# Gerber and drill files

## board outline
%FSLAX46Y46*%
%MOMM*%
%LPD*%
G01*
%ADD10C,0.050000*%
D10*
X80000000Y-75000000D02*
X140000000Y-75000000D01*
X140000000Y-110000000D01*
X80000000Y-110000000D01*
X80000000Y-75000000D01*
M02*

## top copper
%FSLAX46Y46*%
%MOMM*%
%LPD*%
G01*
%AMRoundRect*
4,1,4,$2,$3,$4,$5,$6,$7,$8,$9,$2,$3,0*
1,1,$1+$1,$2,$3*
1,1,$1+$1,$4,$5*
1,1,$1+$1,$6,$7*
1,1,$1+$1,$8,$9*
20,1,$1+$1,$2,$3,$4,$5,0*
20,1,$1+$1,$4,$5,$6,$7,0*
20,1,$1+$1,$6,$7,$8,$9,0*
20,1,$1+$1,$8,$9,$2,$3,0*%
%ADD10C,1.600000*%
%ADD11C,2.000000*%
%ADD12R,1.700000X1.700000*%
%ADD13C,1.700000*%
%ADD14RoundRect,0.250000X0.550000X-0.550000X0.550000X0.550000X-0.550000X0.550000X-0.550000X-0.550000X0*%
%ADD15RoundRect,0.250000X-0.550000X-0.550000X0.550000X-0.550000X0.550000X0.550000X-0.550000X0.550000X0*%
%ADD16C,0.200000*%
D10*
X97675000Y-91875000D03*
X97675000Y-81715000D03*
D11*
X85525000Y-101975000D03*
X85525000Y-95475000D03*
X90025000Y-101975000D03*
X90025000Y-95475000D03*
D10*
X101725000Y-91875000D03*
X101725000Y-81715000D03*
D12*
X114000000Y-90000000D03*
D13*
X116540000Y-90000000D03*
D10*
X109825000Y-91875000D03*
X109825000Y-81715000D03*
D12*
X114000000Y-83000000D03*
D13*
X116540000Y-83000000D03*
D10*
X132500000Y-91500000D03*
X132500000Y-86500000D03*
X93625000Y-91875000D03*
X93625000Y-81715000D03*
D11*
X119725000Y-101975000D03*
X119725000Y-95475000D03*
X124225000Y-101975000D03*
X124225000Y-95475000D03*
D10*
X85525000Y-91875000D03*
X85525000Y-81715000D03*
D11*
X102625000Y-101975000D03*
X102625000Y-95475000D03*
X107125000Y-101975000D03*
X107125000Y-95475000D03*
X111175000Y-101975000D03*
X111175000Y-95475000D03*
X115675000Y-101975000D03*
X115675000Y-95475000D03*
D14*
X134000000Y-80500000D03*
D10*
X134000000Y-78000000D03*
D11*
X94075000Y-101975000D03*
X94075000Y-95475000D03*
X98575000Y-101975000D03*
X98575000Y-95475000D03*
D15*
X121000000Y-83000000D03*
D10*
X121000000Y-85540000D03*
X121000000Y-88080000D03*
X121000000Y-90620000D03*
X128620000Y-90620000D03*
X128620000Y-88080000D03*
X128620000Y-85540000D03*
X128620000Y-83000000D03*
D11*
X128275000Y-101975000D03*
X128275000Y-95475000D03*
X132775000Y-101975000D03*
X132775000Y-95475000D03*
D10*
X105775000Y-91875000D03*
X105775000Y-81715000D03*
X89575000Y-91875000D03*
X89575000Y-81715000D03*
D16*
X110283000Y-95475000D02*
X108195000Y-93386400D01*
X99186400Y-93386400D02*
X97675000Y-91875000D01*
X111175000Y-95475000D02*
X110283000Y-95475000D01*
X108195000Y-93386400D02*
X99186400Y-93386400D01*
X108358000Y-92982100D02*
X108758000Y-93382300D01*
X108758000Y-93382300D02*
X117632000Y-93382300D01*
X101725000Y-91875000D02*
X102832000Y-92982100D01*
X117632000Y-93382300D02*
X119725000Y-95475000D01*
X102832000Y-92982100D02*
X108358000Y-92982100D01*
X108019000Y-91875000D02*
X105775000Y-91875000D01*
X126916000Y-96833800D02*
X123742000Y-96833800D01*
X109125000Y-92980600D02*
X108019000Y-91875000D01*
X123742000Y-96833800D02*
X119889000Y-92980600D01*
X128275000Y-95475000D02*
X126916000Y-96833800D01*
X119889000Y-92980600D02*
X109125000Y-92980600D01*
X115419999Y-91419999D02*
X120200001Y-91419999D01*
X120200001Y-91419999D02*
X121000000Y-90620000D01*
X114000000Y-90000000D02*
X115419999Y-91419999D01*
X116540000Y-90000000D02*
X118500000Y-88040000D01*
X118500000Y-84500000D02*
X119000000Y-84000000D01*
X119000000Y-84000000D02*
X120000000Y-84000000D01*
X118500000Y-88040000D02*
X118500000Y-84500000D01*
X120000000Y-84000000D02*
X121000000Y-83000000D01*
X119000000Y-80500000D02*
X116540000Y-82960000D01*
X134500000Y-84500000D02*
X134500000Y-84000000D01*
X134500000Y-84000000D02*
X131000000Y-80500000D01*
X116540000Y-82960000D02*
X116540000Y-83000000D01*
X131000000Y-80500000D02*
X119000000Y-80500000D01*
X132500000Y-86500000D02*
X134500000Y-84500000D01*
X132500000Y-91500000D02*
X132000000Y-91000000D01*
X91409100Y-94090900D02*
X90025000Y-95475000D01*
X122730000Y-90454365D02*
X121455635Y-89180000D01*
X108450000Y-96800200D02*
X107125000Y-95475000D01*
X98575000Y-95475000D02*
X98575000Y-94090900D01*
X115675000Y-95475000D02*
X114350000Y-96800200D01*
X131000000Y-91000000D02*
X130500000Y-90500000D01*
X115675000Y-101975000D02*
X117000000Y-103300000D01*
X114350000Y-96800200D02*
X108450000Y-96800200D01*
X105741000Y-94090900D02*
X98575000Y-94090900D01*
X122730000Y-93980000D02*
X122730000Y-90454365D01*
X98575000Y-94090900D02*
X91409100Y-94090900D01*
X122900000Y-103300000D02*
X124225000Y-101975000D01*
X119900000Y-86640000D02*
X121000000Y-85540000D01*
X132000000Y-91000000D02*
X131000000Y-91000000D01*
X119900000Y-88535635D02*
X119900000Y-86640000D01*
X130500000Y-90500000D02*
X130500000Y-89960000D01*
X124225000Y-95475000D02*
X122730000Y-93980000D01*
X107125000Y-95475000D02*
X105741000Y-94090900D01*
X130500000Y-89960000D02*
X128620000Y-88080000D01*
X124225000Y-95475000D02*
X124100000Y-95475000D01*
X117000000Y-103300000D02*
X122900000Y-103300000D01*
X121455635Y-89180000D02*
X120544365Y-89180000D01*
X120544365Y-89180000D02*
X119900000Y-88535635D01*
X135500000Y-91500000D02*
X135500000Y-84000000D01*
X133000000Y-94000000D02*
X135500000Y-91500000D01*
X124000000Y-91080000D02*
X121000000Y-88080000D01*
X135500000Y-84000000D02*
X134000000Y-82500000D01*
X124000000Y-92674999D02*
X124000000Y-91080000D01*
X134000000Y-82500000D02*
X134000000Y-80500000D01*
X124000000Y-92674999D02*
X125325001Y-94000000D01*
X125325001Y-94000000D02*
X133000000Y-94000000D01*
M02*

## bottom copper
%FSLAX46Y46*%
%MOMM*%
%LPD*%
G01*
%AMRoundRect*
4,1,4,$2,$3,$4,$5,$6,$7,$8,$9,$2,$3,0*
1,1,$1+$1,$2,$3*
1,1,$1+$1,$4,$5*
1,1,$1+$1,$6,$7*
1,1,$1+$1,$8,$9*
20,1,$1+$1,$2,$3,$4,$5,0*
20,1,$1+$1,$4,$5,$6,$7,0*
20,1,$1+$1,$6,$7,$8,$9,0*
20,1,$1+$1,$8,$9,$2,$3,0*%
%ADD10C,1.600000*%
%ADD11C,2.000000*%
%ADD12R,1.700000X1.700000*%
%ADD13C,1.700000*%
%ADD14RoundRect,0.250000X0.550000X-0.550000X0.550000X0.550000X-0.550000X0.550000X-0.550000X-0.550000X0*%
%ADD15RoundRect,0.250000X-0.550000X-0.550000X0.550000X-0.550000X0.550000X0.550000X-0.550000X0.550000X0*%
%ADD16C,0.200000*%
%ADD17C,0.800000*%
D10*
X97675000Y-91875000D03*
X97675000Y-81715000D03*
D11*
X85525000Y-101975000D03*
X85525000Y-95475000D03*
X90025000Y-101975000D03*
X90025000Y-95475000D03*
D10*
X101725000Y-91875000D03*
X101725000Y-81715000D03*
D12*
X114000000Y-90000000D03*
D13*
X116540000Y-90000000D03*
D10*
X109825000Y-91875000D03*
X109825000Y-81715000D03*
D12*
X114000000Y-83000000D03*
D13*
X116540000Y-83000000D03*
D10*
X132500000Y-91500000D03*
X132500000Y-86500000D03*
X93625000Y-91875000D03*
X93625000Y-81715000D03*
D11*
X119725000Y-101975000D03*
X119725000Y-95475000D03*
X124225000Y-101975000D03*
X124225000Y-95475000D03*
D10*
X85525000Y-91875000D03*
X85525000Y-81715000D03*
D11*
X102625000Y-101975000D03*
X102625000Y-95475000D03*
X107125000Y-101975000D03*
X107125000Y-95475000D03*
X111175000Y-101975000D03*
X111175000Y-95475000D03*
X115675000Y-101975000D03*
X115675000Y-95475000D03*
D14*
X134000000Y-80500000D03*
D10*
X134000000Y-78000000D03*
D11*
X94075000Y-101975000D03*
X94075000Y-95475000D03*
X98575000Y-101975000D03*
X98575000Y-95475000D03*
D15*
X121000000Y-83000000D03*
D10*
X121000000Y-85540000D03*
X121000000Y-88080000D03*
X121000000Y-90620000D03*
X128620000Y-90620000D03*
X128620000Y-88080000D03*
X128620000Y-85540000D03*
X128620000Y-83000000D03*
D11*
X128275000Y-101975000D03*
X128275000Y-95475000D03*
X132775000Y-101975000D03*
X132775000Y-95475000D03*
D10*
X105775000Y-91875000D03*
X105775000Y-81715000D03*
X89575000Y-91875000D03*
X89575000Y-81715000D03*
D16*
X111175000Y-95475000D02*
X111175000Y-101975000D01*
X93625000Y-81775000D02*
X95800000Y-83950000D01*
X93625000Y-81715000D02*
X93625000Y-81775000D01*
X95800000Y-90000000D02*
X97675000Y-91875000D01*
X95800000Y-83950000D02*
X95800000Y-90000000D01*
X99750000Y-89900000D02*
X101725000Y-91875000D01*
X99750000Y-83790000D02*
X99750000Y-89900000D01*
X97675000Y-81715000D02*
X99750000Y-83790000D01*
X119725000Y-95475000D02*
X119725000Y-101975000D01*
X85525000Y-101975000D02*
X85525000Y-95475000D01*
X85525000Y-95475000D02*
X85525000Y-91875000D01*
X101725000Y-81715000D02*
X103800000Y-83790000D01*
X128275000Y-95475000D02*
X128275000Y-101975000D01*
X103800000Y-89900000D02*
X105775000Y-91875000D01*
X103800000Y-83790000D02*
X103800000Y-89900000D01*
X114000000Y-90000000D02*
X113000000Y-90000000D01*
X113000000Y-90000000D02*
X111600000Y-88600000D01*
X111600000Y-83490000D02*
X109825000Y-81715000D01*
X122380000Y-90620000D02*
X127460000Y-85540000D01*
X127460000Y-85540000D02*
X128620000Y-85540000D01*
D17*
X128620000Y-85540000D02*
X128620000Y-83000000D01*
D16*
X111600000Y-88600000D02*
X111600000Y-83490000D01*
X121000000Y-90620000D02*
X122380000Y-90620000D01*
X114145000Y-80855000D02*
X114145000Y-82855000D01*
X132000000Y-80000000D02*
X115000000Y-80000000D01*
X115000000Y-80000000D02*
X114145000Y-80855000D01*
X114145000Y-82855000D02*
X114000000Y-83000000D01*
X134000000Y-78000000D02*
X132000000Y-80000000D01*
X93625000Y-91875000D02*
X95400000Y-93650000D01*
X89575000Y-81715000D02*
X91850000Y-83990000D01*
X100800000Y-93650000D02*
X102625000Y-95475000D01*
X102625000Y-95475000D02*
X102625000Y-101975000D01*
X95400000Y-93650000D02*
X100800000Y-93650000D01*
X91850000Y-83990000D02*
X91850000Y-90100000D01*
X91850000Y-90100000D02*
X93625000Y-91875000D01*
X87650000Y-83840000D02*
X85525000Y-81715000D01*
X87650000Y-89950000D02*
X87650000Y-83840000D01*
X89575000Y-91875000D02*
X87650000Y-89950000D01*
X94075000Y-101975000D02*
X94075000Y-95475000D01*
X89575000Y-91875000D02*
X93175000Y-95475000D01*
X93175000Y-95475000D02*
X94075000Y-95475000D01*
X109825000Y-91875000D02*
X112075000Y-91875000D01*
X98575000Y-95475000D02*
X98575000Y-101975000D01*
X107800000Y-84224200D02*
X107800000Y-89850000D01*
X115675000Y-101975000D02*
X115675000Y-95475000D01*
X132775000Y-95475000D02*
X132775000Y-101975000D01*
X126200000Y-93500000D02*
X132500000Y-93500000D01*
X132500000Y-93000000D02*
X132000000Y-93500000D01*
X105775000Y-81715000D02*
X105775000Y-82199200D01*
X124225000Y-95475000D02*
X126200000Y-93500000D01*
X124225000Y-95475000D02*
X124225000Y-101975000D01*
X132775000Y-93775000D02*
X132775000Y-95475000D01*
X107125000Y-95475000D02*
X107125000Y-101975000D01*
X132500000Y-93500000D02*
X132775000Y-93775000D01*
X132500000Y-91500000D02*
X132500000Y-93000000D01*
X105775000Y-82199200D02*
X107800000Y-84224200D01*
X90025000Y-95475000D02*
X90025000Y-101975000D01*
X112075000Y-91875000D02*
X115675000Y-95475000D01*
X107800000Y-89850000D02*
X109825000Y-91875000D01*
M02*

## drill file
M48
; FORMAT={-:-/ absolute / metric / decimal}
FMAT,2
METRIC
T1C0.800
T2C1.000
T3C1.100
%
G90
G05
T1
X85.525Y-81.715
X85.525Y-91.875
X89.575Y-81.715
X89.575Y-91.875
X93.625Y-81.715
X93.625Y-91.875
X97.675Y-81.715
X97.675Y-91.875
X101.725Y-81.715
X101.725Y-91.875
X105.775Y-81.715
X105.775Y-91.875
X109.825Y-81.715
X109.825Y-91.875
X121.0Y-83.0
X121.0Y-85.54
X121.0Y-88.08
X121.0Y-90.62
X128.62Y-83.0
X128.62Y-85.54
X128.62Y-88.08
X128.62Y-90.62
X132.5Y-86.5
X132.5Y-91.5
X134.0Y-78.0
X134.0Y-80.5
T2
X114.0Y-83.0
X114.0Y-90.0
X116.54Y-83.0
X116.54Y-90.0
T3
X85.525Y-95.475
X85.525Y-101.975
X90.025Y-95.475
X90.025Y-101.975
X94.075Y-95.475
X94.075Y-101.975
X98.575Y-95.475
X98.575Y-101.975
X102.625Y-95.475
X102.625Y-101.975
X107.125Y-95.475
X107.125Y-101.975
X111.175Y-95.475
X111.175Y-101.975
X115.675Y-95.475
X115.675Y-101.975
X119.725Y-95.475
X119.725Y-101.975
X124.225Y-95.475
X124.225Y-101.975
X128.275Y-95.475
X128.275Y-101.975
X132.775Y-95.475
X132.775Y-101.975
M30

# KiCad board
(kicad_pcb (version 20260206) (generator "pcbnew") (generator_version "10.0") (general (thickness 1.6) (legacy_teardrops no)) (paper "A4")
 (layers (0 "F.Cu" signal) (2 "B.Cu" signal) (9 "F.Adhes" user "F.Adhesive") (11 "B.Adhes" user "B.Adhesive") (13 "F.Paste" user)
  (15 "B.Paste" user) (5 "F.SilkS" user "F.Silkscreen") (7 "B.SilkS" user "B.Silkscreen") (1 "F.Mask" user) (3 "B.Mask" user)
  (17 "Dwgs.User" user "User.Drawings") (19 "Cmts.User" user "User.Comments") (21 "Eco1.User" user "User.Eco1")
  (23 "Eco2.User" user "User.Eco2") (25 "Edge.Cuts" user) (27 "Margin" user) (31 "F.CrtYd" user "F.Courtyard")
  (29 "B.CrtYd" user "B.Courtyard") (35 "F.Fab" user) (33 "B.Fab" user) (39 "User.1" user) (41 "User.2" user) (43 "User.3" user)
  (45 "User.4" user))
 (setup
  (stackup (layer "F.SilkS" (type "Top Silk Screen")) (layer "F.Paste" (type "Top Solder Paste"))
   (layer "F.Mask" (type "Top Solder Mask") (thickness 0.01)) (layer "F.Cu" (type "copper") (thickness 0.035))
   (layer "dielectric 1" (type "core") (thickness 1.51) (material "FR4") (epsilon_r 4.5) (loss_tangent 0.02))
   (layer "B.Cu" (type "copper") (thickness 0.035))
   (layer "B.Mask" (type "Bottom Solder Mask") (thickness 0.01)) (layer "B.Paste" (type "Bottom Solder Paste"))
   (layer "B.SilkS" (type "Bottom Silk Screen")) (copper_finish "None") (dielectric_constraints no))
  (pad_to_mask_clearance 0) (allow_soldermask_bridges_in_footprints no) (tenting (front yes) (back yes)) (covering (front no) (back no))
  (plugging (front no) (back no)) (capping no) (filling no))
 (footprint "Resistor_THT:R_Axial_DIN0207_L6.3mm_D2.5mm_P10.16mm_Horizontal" (layer "F.Cu") (at 97.675 91.875 90)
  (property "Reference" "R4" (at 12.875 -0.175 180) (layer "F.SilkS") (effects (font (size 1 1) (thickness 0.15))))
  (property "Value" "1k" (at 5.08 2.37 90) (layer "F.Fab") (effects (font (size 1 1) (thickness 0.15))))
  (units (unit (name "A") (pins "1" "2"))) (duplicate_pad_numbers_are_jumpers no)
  (pad "1" thru_hole circle (at 0 0 90) (size 1.6 1.6) (drill 0.8) (layers "*.Cu" "*.Mask") (remove_unused_layers no) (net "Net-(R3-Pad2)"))
  (pad "2" thru_hole circle (at 10.16 0 90) (size 1.6 1.6) (drill 0.8) (layers "*.Cu" "*.Mask") (remove_unused_layers no)
   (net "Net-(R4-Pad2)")))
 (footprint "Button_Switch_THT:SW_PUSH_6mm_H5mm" (layer "F.Cu") (at 85.525 101.975 90)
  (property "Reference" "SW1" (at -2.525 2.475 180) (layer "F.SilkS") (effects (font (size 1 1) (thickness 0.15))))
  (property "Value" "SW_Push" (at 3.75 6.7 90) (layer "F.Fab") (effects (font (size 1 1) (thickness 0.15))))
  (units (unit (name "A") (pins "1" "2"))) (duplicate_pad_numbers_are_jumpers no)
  (pad "1" thru_hole circle (at 0 0 180) (size 2 2) (drill 1.1) (layers "*.Cu" "*.Mask") (remove_unused_layers no) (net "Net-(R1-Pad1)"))
  (pad "1" thru_hole circle (at 6.5 0 180) (size 2 2) (drill 1.1) (layers "*.Cu" "*.Mask") (remove_unused_layers no) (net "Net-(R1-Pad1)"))
  (pad "2" thru_hole circle (at 0 4.5 180) (size 2 2) (drill 1.1) (layers "*.Cu" "*.Mask") (remove_unused_layers no) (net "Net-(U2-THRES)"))
  (pad "2" thru_hole circle (at 6.5 4.5 180) (size 2 2) (drill 1.1) (layers "*.Cu" "*.Mask") (remove_unused_layers no)
   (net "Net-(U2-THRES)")))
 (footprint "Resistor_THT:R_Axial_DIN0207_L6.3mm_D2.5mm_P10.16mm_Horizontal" (layer "F.Cu") (at 101.725 91.875 90)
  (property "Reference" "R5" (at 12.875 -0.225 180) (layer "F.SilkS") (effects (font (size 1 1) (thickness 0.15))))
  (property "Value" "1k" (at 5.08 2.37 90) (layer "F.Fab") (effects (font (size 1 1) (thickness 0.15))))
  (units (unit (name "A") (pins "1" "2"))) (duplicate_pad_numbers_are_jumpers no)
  (pad "1" thru_hole circle (at 0 0 90) (size 1.6 1.6) (drill 0.8) (layers "*.Cu" "*.Mask") (remove_unused_layers no) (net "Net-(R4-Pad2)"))
  (pad "2" thru_hole circle (at 10.16 0 90) (size 1.6 1.6) (drill 0.8) (layers "*.Cu" "*.Mask") (remove_unused_layers no)
   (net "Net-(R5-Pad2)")))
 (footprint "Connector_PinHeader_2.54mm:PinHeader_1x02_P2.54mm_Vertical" (layer "F.Cu") (at 114 90 90)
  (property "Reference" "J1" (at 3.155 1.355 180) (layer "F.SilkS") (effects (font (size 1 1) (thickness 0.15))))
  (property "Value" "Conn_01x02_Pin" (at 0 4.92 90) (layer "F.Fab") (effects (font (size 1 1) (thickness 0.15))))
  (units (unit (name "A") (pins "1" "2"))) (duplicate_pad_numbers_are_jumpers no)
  (pad "1" thru_hole rect (at 0 0 90) (size 1.7 1.7) (drill 1) (layers "*.Cu" "*.Mask") (remove_unused_layers no) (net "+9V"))
  (pad "2" thru_hole circle (at 0 2.54 90) (size 1.7 1.7) (drill 1) (layers "*.Cu" "*.Mask") (remove_unused_layers no) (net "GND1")))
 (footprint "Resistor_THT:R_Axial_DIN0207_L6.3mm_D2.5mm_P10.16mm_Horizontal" (layer "F.Cu") (at 109.825 91.875 90)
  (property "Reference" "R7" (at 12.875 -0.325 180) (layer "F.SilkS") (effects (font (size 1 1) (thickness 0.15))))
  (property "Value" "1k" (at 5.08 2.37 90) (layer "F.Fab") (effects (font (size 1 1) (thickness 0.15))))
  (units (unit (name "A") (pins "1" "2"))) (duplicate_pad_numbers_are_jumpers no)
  (pad "1" thru_hole circle (at 0 0 90) (size 1.6 1.6) (drill 0.8) (layers "*.Cu" "*.Mask") (remove_unused_layers no) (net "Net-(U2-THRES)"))
  (pad "2" thru_hole circle (at 10.16 0 90) (size 1.6 1.6) (drill 0.8) (layers "*.Cu" "*.Mask") (remove_unused_layers no) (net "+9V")))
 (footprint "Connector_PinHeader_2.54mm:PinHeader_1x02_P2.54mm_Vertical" (layer "F.Cu") (at 114 83 90)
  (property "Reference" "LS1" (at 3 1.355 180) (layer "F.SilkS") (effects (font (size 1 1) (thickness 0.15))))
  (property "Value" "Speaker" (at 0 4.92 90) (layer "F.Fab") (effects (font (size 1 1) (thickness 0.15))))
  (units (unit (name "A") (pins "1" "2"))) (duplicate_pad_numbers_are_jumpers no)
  (pad "1" thru_hole rect (at 0 0 90) (size 1.7 1.7) (drill 1) (layers "*.Cu" "*.Mask") (remove_unused_layers no) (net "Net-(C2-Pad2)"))
  (pad "2" thru_hole circle (at 0 2.54 90) (size 1.7 1.7) (drill 1) (layers "*.Cu" "*.Mask") (remove_unused_layers no) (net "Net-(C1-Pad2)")))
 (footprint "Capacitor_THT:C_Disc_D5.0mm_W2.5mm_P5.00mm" (layer "F.Cu") (at 132.5 91.5 90)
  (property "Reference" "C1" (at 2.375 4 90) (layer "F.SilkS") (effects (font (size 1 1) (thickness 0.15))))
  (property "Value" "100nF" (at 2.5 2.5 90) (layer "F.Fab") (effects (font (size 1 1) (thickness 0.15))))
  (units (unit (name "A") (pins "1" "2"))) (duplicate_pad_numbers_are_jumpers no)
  (pad "1" thru_hole circle (at 0 0 90) (size 1.6 1.6) (drill 0.8) (layers "*.Cu" "*.Mask") (remove_unused_layers no) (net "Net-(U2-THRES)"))
  (pad "2" thru_hole circle (at 5 0 90) (size 1.6 1.6) (drill 0.8) (layers "*.Cu" "*.Mask") (remove_unused_layers no) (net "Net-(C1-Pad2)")))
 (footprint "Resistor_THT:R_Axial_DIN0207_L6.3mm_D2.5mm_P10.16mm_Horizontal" (layer "F.Cu") (at 93.625 91.875 90)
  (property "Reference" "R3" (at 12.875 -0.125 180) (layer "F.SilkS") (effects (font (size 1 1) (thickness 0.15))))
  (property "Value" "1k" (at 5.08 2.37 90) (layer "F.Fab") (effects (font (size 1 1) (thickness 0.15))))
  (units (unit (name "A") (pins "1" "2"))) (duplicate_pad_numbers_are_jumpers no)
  (pad "1" thru_hole circle (at 0 0 90) (size 1.6 1.6) (drill 0.8) (layers "*.Cu" "*.Mask") (remove_unused_layers no) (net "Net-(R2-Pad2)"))
  (pad "2" thru_hole circle (at 10.16 0 90) (size 1.6 1.6) (drill 0.8) (layers "*.Cu" "*.Mask") (remove_unused_layers no)
   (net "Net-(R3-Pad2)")))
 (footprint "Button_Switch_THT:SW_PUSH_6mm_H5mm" (layer "F.Cu") (at 119.725 101.975 90)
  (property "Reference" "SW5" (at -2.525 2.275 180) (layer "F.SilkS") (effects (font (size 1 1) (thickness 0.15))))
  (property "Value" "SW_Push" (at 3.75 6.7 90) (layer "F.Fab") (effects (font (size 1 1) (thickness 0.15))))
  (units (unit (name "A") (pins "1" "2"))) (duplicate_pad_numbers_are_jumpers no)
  (pad "1" thru_hole circle (at 0 0 180) (size 2 2) (drill 1.1) (layers "*.Cu" "*.Mask") (remove_unused_layers no) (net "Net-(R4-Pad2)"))
  (pad "1" thru_hole circle (at 6.5 0 180) (size 2 2) (drill 1.1) (layers "*.Cu" "*.Mask") (remove_unused_layers no) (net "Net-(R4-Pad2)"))
  (pad "2" thru_hole circle (at 0 4.5 180) (size 2 2) (drill 1.1) (layers "*.Cu" "*.Mask") (remove_unused_layers no) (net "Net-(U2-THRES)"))
  (pad "2" thru_hole circle (at 6.5 4.5 180) (size 2 2) (drill 1.1) (layers "*.Cu" "*.Mask") (remove_unused_layers no)
   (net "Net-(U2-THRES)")))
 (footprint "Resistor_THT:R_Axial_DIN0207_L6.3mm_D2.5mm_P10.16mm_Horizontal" (layer "F.Cu") (at 85.525 91.875 90)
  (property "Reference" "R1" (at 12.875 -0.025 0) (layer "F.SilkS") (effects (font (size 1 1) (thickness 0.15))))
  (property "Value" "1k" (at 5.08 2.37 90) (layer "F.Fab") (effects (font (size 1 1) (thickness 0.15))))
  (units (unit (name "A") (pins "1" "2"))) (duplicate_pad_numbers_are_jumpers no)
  (pad "1" thru_hole circle (at 0 0 90) (size 1.6 1.6) (drill 0.8) (layers "*.Cu" "*.Mask") (remove_unused_layers no) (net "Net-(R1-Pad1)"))
  (pad "2" thru_hole circle (at 10.16 0 90) (size 1.6 1.6) (drill 0.8) (layers "*.Cu" "*.Mask") (remove_unused_layers no)
   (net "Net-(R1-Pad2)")))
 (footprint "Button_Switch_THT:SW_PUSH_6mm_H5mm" (layer "F.Cu") (at 102.625 101.975 90)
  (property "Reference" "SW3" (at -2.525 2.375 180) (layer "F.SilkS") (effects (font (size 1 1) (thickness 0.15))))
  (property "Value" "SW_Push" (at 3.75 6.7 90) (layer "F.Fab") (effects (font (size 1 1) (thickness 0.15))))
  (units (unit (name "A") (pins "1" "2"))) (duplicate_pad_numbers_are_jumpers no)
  (pad "1" thru_hole circle (at 0 0 180) (size 2 2) (drill 1.1) (layers "*.Cu" "*.Mask") (remove_unused_layers no) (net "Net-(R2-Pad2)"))
  (pad "1" thru_hole circle (at 6.5 0 180) (size 2 2) (drill 1.1) (layers "*.Cu" "*.Mask") (remove_unused_layers no) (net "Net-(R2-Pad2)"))
  (pad "2" thru_hole circle (at 0 4.5 180) (size 2 2) (drill 1.1) (layers "*.Cu" "*.Mask") (remove_unused_layers no) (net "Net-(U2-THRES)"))
  (pad "2" thru_hole circle (at 6.5 4.5 180) (size 2 2) (drill 1.1) (layers "*.Cu" "*.Mask") (remove_unused_layers no)
   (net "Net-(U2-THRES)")))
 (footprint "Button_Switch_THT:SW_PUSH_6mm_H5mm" (layer "F.Cu") (at 111.175 101.975 90)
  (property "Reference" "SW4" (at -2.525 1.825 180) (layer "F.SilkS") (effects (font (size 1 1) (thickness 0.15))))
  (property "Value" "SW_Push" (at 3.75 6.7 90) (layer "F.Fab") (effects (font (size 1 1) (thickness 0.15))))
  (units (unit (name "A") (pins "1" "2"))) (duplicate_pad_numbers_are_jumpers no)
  (pad "1" thru_hole circle (at 0 0 180) (size 2 2) (drill 1.1) (layers "*.Cu" "*.Mask") (remove_unused_layers no) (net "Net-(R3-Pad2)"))
  (pad "1" thru_hole circle (at 6.5 0 180) (size 2 2) (drill 1.1) (layers "*.Cu" "*.Mask") (remove_unused_layers no) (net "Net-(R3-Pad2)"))
  (pad "2" thru_hole circle (at 0 4.5 180) (size 2 2) (drill 1.1) (layers "*.Cu" "*.Mask") (remove_unused_layers no) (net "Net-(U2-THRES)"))
  (pad "2" thru_hole circle (at 6.5 4.5 180) (size 2 2) (drill 1.1) (layers "*.Cu" "*.Mask") (remove_unused_layers no)
   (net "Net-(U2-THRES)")))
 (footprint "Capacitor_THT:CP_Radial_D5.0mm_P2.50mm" (layer "F.Cu") (at 134 80.5 90)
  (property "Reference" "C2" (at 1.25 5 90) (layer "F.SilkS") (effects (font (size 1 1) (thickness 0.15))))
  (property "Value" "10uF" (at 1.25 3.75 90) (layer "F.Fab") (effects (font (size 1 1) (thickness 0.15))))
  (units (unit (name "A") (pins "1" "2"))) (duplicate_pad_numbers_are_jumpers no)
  (pad "1" thru_hole roundrect (at 0 0 90) (size 1.6 1.6) (drill 0.8) (layers "*.Cu" "*.Mask") (remove_unused_layers no)
   (roundrect_rratio 0.15625) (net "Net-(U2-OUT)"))
  (pad "2" thru_hole circle (at 2.5 0 90) (size 1.6 1.6) (drill 0.8) (layers "*.Cu" "*.Mask") (remove_unused_layers no)
   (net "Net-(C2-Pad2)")))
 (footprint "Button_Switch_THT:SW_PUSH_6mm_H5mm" (layer "F.Cu") (at 94.075 101.975 90)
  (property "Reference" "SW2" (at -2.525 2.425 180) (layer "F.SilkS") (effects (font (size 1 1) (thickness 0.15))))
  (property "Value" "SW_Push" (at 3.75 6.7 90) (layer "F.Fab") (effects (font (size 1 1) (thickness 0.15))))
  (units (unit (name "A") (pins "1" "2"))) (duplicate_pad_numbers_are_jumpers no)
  (pad "1" thru_hole circle (at 0 0 180) (size 2 2) (drill 1.1) (layers "*.Cu" "*.Mask") (remove_unused_layers no) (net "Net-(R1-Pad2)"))
  (pad "1" thru_hole circle (at 6.5 0 180) (size 2 2) (drill 1.1) (layers "*.Cu" "*.Mask") (remove_unused_layers no) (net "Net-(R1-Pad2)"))
  (pad "2" thru_hole circle (at 0 4.5 180) (size 2 2) (drill 1.1) (layers "*.Cu" "*.Mask") (remove_unused_layers no) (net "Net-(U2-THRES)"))
  (pad "2" thru_hole circle (at 6.5 4.5 180) (size 2 2) (drill 1.1) (layers "*.Cu" "*.Mask") (remove_unused_layers no)
   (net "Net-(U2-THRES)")))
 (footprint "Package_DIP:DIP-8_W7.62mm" (layer "F.Cu") (at 121 83)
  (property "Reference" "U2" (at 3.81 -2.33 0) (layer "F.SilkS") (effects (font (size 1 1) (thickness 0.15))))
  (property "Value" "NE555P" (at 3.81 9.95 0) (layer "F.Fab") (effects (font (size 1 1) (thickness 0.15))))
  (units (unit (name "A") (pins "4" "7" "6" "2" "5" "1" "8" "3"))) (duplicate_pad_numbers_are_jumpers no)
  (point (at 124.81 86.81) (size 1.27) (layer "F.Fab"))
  (pad "1" thru_hole roundrect (at 0 0) (size 1.6 1.6) (drill 0.8) (layers "*.Cu" "*.Mask") (remove_unused_layers no)
   (roundrect_rratio 0.15625) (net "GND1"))
  (pad "2" thru_hole circle (at 0 2.54) (size 1.6 1.6) (drill 0.8) (layers "*.Cu" "*.Mask") (remove_unused_layers no) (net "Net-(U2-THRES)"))
  (pad "3" thru_hole circle (at 0 5.08) (size 1.6 1.6) (drill 0.8) (layers "*.Cu" "*.Mask") (remove_unused_layers no) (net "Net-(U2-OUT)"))
  (pad "4" thru_hole circle (at 0 7.62) (size 1.6 1.6) (drill 0.8) (layers "*.Cu" "*.Mask") (remove_unused_layers no) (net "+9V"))
  (pad "5" thru_hole circle (at 7.62 7.62) (size 1.6 1.6) (drill 0.8) (layers "*.Cu" "*.Mask") (remove_unused_layers no)
   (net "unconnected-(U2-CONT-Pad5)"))
  (pad "6" thru_hole circle (at 7.62 5.08) (size 1.6 1.6) (drill 0.8) (layers "*.Cu" "*.Mask") (remove_unused_layers no)
   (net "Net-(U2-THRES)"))
  (pad "7" thru_hole circle (at 7.62 2.54) (size 1.6 1.6) (drill 0.8) (layers "*.Cu" "*.Mask") (remove_unused_layers no) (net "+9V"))
  (pad "8" thru_hole circle (at 7.62 0) (size 1.6 1.6) (drill 0.8) (layers "*.Cu" "*.Mask") (remove_unused_layers no) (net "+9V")))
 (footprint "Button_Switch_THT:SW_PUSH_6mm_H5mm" (layer "F.Cu") (at 128.275 101.975 90)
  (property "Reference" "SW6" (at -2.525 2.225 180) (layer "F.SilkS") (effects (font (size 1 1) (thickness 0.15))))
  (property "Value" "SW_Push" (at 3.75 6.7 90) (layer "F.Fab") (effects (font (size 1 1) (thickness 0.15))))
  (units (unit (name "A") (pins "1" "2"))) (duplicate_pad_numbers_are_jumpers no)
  (pad "1" thru_hole circle (at 0 0 180) (size 2 2) (drill 1.1) (layers "*.Cu" "*.Mask") (remove_unused_layers no) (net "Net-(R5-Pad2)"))
  (pad "1" thru_hole circle (at 6.5 0 180) (size 2 2) (drill 1.1) (layers "*.Cu" "*.Mask") (remove_unused_layers no) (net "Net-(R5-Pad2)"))
  (pad "2" thru_hole circle (at 0 4.5 180) (size 2 2) (drill 1.1) (layers "*.Cu" "*.Mask") (remove_unused_layers no) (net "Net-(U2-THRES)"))
  (pad "2" thru_hole circle (at 6.5 4.5 180) (size 2 2) (drill 1.1) (layers "*.Cu" "*.Mask") (remove_unused_layers no)
   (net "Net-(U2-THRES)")))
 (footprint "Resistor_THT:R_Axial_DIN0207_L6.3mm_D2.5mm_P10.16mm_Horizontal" (layer "F.Cu") (at 105.775 91.875 90)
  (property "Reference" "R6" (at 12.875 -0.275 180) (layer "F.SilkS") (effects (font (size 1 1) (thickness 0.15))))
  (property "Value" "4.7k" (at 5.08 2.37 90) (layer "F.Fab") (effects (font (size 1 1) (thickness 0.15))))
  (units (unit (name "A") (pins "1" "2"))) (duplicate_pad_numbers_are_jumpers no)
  (pad "1" thru_hole circle (at 0 0 90) (size 1.6 1.6) (drill 0.8) (layers "*.Cu" "*.Mask") (remove_unused_layers no) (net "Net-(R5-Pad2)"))
  (pad "2" thru_hole circle (at 10.16 0 90) (size 1.6 1.6) (drill 0.8) (layers "*.Cu" "*.Mask") (remove_unused_layers no)
   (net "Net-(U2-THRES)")))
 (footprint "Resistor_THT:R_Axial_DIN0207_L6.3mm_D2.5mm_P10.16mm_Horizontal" (layer "F.Cu") (at 89.575 91.875 90)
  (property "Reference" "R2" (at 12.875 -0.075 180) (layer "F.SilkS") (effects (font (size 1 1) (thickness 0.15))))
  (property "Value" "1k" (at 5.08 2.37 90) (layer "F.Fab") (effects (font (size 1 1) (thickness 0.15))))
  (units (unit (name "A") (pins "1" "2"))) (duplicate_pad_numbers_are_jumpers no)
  (pad "1" thru_hole circle (at 0 0 90) (size 1.6 1.6) (drill 0.8) (layers "*.Cu" "*.Mask") (remove_unused_layers no) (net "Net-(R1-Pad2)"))
  (pad "2" thru_hole circle (at 10.16 0 90) (size 1.6 1.6) (drill 0.8) (layers "*.Cu" "*.Mask") (remove_unused_layers no)
   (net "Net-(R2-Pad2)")))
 (gr_rect (start 80 75) (end 140 110) (stroke (width 0.05) (type default)) (fill no) (layer "Edge.Cuts"))
 (segment (start 110.283 95.475) (end 108.195 93.3864) (width 0.2) (layer "F.Cu") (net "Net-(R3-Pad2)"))
 (segment (start 99.1864 93.3864) (end 97.675 91.875) (width 0.2) (layer "F.Cu") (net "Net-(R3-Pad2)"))
 (segment (start 111.175 95.475) (end 110.283 95.475) (width 0.2) (layer "F.Cu") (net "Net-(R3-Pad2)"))
 (segment (start 108.195 93.3864) (end 99.1864 93.3864) (width 0.2) (layer "F.Cu") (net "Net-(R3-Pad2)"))
 (segment (start 111.175 95.475) (end 111.175 101.975) (width 0.2) (layer "B.Cu") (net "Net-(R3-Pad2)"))
 (segment (start 93.625 81.775) (end 95.8 83.95) (width 0.2) (layer "B.Cu") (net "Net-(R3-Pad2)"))
 (segment (start 93.625 81.715) (end 93.625 81.775) (width 0.2) (layer "B.Cu") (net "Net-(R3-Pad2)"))
 (segment (start 95.8 90) (end 97.675 91.875) (width 0.2) (layer "B.Cu") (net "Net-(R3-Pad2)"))
 (segment (start 95.8 83.95) (end 95.8 90) (width 0.2) (layer "B.Cu") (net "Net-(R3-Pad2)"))
 (segment (start 108.358 92.9821) (end 108.758 93.3823) (width 0.2) (layer "F.Cu") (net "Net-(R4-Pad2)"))
 (segment (start 108.758 93.3823) (end 117.632 93.3823) (width 0.2) (layer "F.Cu") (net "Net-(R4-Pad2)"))
 (segment (start 101.725 91.875) (end 102.832 92.9821) (width 0.2) (layer "F.Cu") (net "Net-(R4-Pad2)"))
 (segment (start 117.632 93.3823) (end 119.725 95.475) (width 0.2) (layer "F.Cu") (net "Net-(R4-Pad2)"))
 (segment (start 102.832 92.9821) (end 108.358 92.9821) (width 0.2) (layer "F.Cu") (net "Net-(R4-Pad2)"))
 (segment (start 99.75 89.9) (end 101.725 91.875) (width 0.2) (layer "B.Cu") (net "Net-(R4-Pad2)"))
 (segment (start 99.75 83.79) (end 99.75 89.9) (width 0.2) (layer "B.Cu") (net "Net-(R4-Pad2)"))
 (segment (start 97.675 81.715) (end 99.75 83.79) (width 0.2) (layer "B.Cu") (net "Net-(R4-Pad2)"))
 (segment (start 119.725 95.475) (end 119.725 101.975) (width 0.2) (layer "B.Cu") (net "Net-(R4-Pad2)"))
 (segment (start 85.525 101.975) (end 85.525 95.475) (width 0.2) (layer "B.Cu") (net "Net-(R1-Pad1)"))
 (segment (start 85.525 95.475) (end 85.525 91.875) (width 0.2) (layer "B.Cu") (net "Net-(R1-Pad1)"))
 (segment (start 108.019 91.875) (end 105.775 91.875) (width 0.2) (layer "F.Cu") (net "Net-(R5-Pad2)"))
 (segment (start 126.916 96.8338) (end 123.742 96.8338) (width 0.2) (layer "F.Cu") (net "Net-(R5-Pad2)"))
 (segment (start 109.125 92.9806) (end 108.019 91.875) (width 0.2) (layer "F.Cu") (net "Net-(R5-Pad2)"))
 (segment (start 123.742 96.8338) (end 119.889 92.9806) (width 0.2) (layer "F.Cu") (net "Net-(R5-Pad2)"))
 (segment (start 128.275 95.475) (end 126.916 96.8338) (width 0.2) (layer "F.Cu") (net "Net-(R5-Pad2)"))
 (segment (start 119.889 92.9806) (end 109.125 92.9806) (width 0.2) (layer "F.Cu") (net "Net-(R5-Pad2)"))
 (segment (start 101.725 81.715) (end 103.8 83.79) (width 0.2) (layer "B.Cu") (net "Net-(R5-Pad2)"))
 (segment (start 128.275 95.475) (end 128.275 101.975) (width 0.2) (layer "B.Cu") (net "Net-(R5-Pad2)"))
 (segment (start 103.8 89.9) (end 105.775 91.875) (width 0.2) (layer "B.Cu") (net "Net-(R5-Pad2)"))
 (segment (start 103.8 83.79) (end 103.8 89.9) (width 0.2) (layer "B.Cu") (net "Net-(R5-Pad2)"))
 (segment (start 115.419999 91.419999) (end 120.200001 91.419999) (width 0.2) (layer "F.Cu") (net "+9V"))
 (segment (start 120.200001 91.419999) (end 121 90.62) (width 0.2) (layer "F.Cu") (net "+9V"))
 (segment (start 114 90) (end 115.419999 91.419999) (width 0.2) (layer "F.Cu") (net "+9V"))
 (segment (start 114 90) (end 113 90) (width 0.2) (layer "B.Cu") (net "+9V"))
 (segment (start 113 90) (end 111.6 88.6) (width 0.2) (layer "B.Cu") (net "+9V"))
 (segment (start 111.6 83.49) (end 109.825 81.715) (width 0.2) (layer "B.Cu") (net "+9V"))
 (segment (start 122.38 90.62) (end 127.46 85.54) (width 0.2) (layer "B.Cu") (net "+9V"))
 (segment (start 127.46 85.54) (end 128.62 85.54) (width 0.2) (layer "B.Cu") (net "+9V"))
 (segment (start 128.62 85.54) (end 128.62 83) (width 0.8) (layer "B.Cu") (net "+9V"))
 (segment (start 111.6 88.6) (end 111.6 83.49) (width 0.2) (layer "B.Cu") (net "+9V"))
 (segment (start 121 90.62) (end 122.38 90.62) (width 0.2) (layer "B.Cu") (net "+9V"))
 (segment (start 116.54 90) (end 118.5 88.04) (width 0.2) (layer "F.Cu") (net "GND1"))
 (segment (start 118.5 84.5) (end 119 84) (width 0.2) (layer "F.Cu") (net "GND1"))
 (segment (start 119 84) (end 120 84) (width 0.2) (layer "F.Cu") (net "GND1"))
 (segment (start 118.5 88.04) (end 118.5 84.5) (width 0.2) (layer "F.Cu") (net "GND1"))
 (segment (start 120 84) (end 121 83) (width 0.2) (layer "F.Cu") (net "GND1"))
 (segment (start 114.145 80.855) (end 114.145 82.855) (width 0.2) (layer "B.Cu") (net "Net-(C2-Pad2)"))
 (segment (start 132 80) (end 115 80) (width 0.2) (layer "B.Cu") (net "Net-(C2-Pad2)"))
 (segment (start 115 80) (end 114.145 80.855) (width 0.2) (layer "B.Cu") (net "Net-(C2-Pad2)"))
 (segment (start 114.145 82.855) (end 114 83) (width 0.2) (layer "B.Cu") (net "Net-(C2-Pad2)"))
 (segment (start 134 78) (end 132 80) (width 0.2) (layer "B.Cu") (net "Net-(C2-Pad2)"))
 (segment (start 119 80.5) (end 116.54 82.96) (width 0.2) (layer "F.Cu") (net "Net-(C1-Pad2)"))
 (segment (start 134.5 84.5) (end 134.5 84) (width 0.2) (layer "F.Cu") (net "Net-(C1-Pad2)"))
 (segment (start 134.5 84) (end 131 80.5) (width 0.2) (layer "F.Cu") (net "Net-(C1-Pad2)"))
 (segment (start 116.54 82.96) (end 116.54 83) (width 0.2) (layer "F.Cu") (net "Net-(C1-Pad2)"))
 (segment (start 131 80.5) (end 119 80.5) (width 0.2) (layer "F.Cu") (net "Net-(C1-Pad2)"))
 (segment (start 132.5 86.5) (end 134.5 84.5) (width 0.2) (layer "F.Cu") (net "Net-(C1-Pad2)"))
 (segment (start 93.625 91.875) (end 95.4 93.65) (width 0.2) (layer "B.Cu") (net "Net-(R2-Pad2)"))
 (segment (start 89.575 81.715) (end 91.85 83.99) (width 0.2) (layer "B.Cu") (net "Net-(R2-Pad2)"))
 (segment (start 100.8 93.65) (end 102.625 95.475) (width 0.2) (layer "B.Cu") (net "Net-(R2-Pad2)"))
 (segment (start 102.625 95.475) (end 102.625 101.975) (width 0.2) (layer "B.Cu") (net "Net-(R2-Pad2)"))
 (segment (start 95.4 93.65) (end 100.8 93.65) (width 0.2) (layer "B.Cu") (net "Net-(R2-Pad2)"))
 (segment (start 91.85 83.99) (end 91.85 90.1) (width 0.2) (layer "B.Cu") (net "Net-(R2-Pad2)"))
 (segment (start 91.85 90.1) (end 93.625 91.875) (width 0.2) (layer "B.Cu") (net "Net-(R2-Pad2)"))
 (segment (start 87.65 83.84) (end 85.525 81.715) (width 0.2) (layer "B.Cu") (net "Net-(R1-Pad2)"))
 (segment (start 87.65 89.95) (end 87.65 83.84) (width 0.2) (layer "B.Cu") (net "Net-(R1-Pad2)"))
 (segment (start 89.575 91.875) (end 87.65 89.95) (width 0.2) (layer "B.Cu") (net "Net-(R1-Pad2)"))
 (segment (start 94.075 101.975) (end 94.075 95.475) (width 0.2) (layer "B.Cu") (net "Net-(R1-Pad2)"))
 (segment (start 89.575 91.875) (end 93.175 95.475) (width 0.2) (layer "B.Cu") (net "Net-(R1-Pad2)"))
 (segment (start 93.175 95.475) (end 94.075 95.475) (width 0.2) (layer "B.Cu") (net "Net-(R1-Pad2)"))
 (segment (start 132.5 91.5) (end 132 91) (width 0.2) (layer "F.Cu") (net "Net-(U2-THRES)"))
 (segment (start 91.4091 94.0909) (end 90.025 95.475) (width 0.2) (layer "F.Cu") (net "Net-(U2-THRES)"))
 (segment (start 122.73 90.454365) (end 121.455635 89.18) (width 0.2) (layer "F.Cu") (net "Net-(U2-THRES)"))
 (segment (start 108.45 96.8002) (end 107.125 95.475) (width 0.2) (layer "F.Cu") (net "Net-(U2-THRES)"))
 (segment (start 98.575 95.475) (end 98.575 94.0909) (width 0.2) (layer "F.Cu") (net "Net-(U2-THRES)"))
 (segment (start 115.675 95.475) (end 114.35 96.8002) (width 0.2) (layer "F.Cu") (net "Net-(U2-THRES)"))
 (segment (start 131 91) (end 130.5 90.5) (width 0.2) (layer "F.Cu") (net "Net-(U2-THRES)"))
 (segment (start 115.675 101.975) (end 117 103.3) (width 0.2) (layer "F.Cu") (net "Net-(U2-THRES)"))
 (segment (start 114.35 96.8002) (end 108.45 96.8002) (width 0.2) (layer "F.Cu") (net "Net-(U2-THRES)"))
 (segment (start 105.741 94.0909) (end 98.575 94.0909) (width 0.2) (layer "F.Cu") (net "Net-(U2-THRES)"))
 (segment (start 122.73 93.98) (end 122.73 90.454365) (width 0.2) (layer "F.Cu") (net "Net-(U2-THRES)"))
 (segment (start 98.575 94.0909) (end 91.4091 94.0909) (width 0.2) (layer "F.Cu") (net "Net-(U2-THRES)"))
 (segment (start 122.9 103.3) (end 124.225 101.975) (width 0.2) (layer "F.Cu") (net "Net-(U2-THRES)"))
 (segment (start 119.9 86.64) (end 121 85.54) (width 0.2) (layer "F.Cu") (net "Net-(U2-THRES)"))
 (segment (start 132 91) (end 131 91) (width 0.2) (layer "F.Cu") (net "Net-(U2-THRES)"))
 (segment (start 119.9 88.535635) (end 119.9 86.64) (width 0.2) (layer "F.Cu") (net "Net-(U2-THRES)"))
 (segment (start 130.5 90.5) (end 130.5 89.96) (width 0.2) (layer "F.Cu") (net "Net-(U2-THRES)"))
 (segment (start 124.225 95.475) (end 122.73 93.98) (width 0.2) (layer "F.Cu") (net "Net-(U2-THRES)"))
 (segment (start 107.125 95.475) (end 105.741 94.0909) (width 0.2) (layer "F.Cu") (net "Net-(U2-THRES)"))
 (segment (start 130.5 89.96) (end 128.62 88.08) (width 0.2) (layer "F.Cu") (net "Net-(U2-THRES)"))
 (segment (start 124.225 95.475) (end 124.1 95.475) (width 0.2) (layer "F.Cu") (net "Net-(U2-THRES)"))
 (segment (start 117 103.3) (end 122.9 103.3) (width 0.2) (layer "F.Cu") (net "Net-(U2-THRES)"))
 (segment (start 121.455635 89.18) (end 120.544365 89.18) (width 0.2) (layer "F.Cu") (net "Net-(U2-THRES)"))
 (segment (start 120.544365 89.18) (end 119.9 88.535635) (width 0.2) (layer "F.Cu") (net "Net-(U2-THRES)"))
 (segment (start 109.825 91.875) (end 112.075 91.875) (width 0.2) (layer "B.Cu") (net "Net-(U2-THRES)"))
 (segment (start 98.575 95.475) (end 98.575 101.975) (width 0.2) (layer "B.Cu") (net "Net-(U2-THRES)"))
 (segment (start 107.8 84.2242) (end 107.8 89.85) (width 0.2) (layer "B.Cu") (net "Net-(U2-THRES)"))
 (segment (start 115.675 101.975) (end 115.675 95.475) (width 0.2) (layer "B.Cu") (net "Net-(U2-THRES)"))
 (segment (start 132.775 95.475) (end 132.775 101.975) (width 0.2) (layer "B.Cu") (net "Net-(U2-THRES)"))
 (segment (start 126.2 93.5) (end 132.5 93.5) (width 0.2) (layer "B.Cu") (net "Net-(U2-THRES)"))
 (segment (start 132.5 93) (end 132 93.5) (width 0.2) (layer "B.Cu") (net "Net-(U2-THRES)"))
 (segment (start 105.775 81.715) (end 105.775 82.1992) (width 0.2) (layer "B.Cu") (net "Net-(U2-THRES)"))
 (segment (start 124.225 95.475) (end 126.2 93.5) (width 0.2) (layer "B.Cu") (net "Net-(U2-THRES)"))
 (segment (start 124.225 95.475) (end 124.225 101.975) (width 0.2) (layer "B.Cu") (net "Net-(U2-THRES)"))
 (segment (start 132.775 93.775) (end 132.775 95.475) (width 0.2) (layer "B.Cu") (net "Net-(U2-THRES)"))
 (segment (start 107.125 95.475) (end 107.125 101.975) (width 0.2) (layer "B.Cu") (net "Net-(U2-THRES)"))
 (segment (start 132.5 93.5) (end 132.775 93.775) (width 0.2) (layer "B.Cu") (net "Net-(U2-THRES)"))
 (segment (start 132.5 91.5) (end 132.5 93) (width 0.2) (layer "B.Cu") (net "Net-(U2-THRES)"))
 (segment (start 105.775 82.1992) (end 107.8 84.2242) (width 0.2) (layer "B.Cu") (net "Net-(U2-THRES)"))
 (segment (start 90.025 95.475) (end 90.025 101.975) (width 0.2) (layer "B.Cu") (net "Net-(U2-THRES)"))
 (segment (start 112.075 91.875) (end 115.675 95.475) (width 0.2) (layer "B.Cu") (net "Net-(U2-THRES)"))
 (segment (start 107.8 89.85) (end 109.825 91.875) (width 0.2) (layer "B.Cu") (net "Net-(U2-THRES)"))
 (segment (start 135.5 91.5) (end 135.5 84) (width 0.2) (layer "F.Cu") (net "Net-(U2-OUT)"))
 (segment (start 133 94) (end 135.5 91.5) (width 0.2) (layer "F.Cu") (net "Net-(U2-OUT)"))
 (segment (start 124 91.08) (end 121 88.08) (width 0.2) (layer "F.Cu") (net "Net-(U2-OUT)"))
 (segment (start 135.5 84) (end 134 82.5) (width 0.2) (layer "F.Cu") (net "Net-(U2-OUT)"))
 (segment (start 124 92.674999) (end 124 91.08) (width 0.2) (layer "F.Cu") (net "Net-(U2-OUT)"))
 (segment (start 134 82.5) (end 134 80.5) (width 0.2) (layer "F.Cu") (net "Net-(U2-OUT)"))
 (segment (start 124 92.674999) (end 125.325001 94) (width 0.2) (layer "F.Cu") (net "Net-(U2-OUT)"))
 (segment (start 125.325001 94) (end 133 94) (width 0.2) (layer "F.Cu") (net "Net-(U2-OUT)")))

